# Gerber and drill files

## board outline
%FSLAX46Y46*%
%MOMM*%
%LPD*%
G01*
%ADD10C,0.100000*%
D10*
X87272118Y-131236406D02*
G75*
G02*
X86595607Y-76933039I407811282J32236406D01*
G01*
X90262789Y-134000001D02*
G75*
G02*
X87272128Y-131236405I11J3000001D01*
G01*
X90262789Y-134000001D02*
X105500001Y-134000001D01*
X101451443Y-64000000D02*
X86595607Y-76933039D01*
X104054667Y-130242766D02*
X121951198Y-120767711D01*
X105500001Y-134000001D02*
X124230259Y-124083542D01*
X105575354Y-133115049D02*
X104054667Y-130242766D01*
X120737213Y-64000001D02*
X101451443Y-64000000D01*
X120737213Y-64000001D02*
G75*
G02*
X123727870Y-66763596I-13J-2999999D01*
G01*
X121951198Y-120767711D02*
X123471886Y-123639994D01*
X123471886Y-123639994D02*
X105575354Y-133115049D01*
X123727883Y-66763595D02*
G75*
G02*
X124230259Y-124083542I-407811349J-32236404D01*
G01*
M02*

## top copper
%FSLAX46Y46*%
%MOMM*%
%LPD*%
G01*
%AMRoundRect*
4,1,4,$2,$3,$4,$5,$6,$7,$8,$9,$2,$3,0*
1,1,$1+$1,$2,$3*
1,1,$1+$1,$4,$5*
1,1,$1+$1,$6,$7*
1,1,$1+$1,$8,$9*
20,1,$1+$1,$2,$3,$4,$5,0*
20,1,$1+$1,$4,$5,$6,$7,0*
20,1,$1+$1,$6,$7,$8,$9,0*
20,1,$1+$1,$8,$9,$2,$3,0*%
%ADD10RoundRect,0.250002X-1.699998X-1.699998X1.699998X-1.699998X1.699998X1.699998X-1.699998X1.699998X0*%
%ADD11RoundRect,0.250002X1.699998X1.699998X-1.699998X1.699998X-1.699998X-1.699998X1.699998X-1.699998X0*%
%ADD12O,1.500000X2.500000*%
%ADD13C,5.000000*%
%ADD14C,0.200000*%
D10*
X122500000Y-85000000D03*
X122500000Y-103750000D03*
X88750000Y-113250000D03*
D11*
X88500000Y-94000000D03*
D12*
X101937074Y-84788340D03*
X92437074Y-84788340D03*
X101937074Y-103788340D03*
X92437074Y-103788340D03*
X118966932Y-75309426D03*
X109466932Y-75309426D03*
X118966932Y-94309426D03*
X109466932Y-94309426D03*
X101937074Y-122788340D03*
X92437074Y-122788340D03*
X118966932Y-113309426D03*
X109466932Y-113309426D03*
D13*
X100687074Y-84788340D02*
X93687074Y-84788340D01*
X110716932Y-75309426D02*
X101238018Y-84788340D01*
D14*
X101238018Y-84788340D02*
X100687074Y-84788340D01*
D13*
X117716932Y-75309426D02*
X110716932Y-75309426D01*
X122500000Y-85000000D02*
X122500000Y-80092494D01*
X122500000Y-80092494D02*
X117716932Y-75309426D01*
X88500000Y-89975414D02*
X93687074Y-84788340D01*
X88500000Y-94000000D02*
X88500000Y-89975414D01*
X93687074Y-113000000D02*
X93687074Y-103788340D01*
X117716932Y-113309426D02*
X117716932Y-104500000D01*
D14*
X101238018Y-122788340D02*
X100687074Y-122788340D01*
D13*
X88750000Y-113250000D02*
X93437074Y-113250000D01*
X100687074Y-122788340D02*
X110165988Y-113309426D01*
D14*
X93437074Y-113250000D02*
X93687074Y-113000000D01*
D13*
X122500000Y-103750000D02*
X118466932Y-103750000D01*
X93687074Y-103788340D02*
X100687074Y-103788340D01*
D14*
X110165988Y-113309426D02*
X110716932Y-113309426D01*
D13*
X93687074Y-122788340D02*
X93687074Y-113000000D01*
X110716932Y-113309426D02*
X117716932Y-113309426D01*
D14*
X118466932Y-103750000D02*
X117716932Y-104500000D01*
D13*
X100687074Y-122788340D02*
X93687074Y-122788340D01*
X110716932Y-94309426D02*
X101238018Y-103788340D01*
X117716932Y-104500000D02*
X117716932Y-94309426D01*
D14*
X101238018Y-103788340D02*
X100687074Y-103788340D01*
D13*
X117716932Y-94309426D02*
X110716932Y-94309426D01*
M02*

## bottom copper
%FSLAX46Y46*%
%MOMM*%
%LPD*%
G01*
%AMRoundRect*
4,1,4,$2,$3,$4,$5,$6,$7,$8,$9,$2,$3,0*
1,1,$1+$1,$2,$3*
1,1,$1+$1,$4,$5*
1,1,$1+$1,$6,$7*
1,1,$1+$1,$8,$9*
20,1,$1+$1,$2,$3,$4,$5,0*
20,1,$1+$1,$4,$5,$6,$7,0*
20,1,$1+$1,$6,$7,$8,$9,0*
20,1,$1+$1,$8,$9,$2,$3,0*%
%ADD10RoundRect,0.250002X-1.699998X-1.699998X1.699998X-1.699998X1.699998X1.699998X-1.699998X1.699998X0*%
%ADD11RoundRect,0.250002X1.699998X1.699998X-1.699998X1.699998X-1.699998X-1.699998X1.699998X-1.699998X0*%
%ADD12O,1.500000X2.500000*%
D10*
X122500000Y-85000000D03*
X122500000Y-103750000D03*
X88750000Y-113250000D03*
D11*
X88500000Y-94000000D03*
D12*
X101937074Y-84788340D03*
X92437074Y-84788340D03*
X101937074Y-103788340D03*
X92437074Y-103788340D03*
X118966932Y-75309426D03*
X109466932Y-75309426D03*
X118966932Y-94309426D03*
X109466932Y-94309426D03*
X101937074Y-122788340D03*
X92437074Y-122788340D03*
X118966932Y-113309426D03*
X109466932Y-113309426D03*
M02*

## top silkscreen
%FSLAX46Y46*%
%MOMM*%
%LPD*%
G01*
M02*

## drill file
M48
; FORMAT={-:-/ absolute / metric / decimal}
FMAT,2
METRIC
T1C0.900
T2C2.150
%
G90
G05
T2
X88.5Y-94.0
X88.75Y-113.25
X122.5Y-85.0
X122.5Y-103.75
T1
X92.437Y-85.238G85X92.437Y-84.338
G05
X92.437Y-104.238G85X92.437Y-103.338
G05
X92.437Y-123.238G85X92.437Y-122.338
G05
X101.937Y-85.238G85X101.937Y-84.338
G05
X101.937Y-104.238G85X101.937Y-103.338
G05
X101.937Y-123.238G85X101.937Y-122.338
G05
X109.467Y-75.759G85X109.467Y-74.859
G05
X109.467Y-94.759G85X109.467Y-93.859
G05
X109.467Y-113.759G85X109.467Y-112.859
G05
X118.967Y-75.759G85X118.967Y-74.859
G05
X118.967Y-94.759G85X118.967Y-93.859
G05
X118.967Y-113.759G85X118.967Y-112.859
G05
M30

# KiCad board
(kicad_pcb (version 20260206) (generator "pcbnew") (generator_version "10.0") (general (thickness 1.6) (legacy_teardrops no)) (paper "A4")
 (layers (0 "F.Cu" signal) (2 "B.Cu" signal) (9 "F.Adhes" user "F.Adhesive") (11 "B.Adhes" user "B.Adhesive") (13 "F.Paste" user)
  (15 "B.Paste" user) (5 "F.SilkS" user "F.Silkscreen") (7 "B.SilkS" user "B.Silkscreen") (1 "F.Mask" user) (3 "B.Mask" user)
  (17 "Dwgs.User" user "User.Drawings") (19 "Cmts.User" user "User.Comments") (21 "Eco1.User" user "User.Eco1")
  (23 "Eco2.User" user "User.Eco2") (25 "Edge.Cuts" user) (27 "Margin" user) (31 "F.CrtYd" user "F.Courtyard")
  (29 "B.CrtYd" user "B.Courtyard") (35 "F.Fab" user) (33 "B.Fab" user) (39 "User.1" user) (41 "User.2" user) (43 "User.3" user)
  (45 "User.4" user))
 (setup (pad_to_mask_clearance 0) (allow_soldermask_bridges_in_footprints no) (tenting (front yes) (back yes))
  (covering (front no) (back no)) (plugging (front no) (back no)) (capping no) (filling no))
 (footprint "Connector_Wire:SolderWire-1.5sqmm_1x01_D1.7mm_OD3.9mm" (layer "F.Cu") (at 122.5 85)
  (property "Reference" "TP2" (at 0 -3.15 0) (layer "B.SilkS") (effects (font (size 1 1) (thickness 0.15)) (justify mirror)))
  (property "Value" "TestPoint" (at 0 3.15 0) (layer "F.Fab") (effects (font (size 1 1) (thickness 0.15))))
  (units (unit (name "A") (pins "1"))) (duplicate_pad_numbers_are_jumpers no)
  (pad "1" thru_hole roundrect (at 0 0) (size 3.9 3.9) (drill 2.15) (layers "*.Cu" "*.Mask") (remove_unused_layers no)
   (roundrect_rratio 0.064103) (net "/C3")))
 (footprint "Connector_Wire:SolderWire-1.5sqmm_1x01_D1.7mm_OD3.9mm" (layer "F.Cu") (at 122.5 103.75)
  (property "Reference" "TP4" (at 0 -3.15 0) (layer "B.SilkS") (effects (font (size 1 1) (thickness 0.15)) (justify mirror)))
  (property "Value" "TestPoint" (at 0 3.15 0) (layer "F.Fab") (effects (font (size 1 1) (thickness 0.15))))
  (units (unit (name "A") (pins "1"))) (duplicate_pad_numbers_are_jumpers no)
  (pad "1" thru_hole roundrect (at 0 0) (size 3.9 3.9) (drill 2.15) (layers "*.Cu" "*.Mask") (remove_unused_layers no)
   (roundrect_rratio 0.064103) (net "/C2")))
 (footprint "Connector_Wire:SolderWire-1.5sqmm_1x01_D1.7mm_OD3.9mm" (layer "F.Cu") (at 88.75 113.25)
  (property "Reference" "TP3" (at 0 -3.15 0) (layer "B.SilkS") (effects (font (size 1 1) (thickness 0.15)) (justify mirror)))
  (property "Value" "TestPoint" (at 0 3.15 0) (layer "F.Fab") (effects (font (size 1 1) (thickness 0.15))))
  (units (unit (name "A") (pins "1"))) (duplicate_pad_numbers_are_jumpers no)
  (pad "1" thru_hole roundrect (at 0 0) (size 3.9 3.9) (drill 2.15) (layers "*.Cu" "*.Mask") (remove_unused_layers no)
   (roundrect_rratio 0.064103) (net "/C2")))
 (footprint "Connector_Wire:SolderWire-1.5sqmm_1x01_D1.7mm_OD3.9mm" (layer "B.Cu") (at 88.5 94 180)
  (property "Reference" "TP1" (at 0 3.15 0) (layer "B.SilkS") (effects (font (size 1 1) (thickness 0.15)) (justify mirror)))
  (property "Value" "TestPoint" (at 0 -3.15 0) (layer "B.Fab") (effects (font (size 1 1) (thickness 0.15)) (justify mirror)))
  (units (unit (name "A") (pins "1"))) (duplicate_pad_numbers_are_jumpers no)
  (pad "1" thru_hole roundrect (at 0 0 180) (size 3.9 3.9) (drill 2.15) (layers "*.Cu" "*.Mask") (remove_unused_layers no)
   (roundrect_rratio 0.064103) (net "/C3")))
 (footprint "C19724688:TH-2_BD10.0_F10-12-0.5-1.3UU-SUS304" (layer "B.Cu") (at 97.187074 84.78834 180)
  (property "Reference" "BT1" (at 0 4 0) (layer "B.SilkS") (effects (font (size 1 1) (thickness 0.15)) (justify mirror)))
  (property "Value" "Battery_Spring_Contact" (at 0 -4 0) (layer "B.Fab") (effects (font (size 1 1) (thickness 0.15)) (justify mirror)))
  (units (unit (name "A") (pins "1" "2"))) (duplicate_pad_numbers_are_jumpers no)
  (pad "1" thru_hole oval (at -4.75 0 180) (size 1.5 2.5) (drill oval 0.900024 1.799996) (layers "*.Cu" "*.Mask") (remove_unused_layers no)
   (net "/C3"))
  (pad "2" thru_hole oval (at 4.75 0 180) (size 1.5 2.5) (drill oval 0.900024 1.799996) (layers "*.Cu" "*.Mask") (remove_unused_layers no)
   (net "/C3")))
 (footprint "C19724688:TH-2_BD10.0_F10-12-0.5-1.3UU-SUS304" (layer "B.Cu") (at 97.187074 103.78834 180)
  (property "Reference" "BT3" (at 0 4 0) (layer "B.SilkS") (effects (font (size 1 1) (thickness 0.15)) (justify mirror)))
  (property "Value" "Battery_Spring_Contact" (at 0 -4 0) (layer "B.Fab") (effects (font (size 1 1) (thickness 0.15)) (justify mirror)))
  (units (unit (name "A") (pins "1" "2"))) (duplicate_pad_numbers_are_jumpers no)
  (pad "1" thru_hole oval (at -4.75 0 180) (size 1.5 2.5) (drill oval 0.900024 1.799996) (layers "*.Cu" "*.Mask") (remove_unused_layers no)
   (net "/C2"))
  (pad "2" thru_hole oval (at 4.75 0 180) (size 1.5 2.5) (drill oval 0.900024 1.799996) (layers "*.Cu" "*.Mask") (remove_unused_layers no)
   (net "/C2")))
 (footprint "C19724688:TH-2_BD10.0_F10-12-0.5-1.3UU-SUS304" (layer "B.Cu") (at 114.216932 75.309426 180)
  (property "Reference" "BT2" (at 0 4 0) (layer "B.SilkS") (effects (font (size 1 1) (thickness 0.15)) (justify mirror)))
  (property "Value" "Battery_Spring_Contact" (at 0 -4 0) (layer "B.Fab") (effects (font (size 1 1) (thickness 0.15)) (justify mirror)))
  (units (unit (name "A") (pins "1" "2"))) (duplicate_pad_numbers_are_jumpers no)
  (pad "1" thru_hole oval (at -4.75 0 180) (size 1.5 2.5) (drill oval 0.900024 1.799996) (layers "*.Cu" "*.Mask") (remove_unused_layers no)
   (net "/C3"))
  (pad "2" thru_hole oval (at 4.75 0 180) (size 1.5 2.5) (drill oval 0.900024 1.799996) (layers "*.Cu" "*.Mask") (remove_unused_layers no)
   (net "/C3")))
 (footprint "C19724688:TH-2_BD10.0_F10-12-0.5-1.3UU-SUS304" (layer "B.Cu") (at 114.216932 94.309426 180)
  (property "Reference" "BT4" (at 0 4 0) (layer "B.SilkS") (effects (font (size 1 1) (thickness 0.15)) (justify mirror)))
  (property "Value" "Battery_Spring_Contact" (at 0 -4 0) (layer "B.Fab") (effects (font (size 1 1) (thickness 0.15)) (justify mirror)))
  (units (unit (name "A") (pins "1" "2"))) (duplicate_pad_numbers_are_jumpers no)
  (pad "1" thru_hole oval (at -4.75 0 180) (size 1.5 2.5) (drill oval 0.900024 1.799996) (layers "*.Cu" "*.Mask") (remove_unused_layers no)
   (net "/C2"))
  (pad "2" thru_hole oval (at 4.75 0 180) (size 1.5 2.5) (drill oval 0.900024 1.799996) (layers "*.Cu" "*.Mask") (remove_unused_layers no)
   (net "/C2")))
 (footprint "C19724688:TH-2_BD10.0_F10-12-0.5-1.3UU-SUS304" (layer "B.Cu") (at 97.187074 122.78834 180)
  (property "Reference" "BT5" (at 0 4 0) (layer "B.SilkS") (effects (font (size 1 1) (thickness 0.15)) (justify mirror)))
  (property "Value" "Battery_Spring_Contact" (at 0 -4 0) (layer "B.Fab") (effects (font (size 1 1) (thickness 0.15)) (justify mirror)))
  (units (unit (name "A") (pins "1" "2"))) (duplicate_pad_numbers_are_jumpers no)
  (pad "1" thru_hole oval (at -4.75 0 180) (size 1.5 2.5) (drill oval 0.900024 1.799996) (layers "*.Cu" "*.Mask") (remove_unused_layers no)
   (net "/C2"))
  (pad "2" thru_hole oval (at 4.75 0 180) (size 1.5 2.5) (drill oval 0.900024 1.799996) (layers "*.Cu" "*.Mask") (remove_unused_layers no)
   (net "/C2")))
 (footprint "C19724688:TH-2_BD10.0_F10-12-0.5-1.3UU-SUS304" (layer "B.Cu") (at 114.216932 113.309426 180)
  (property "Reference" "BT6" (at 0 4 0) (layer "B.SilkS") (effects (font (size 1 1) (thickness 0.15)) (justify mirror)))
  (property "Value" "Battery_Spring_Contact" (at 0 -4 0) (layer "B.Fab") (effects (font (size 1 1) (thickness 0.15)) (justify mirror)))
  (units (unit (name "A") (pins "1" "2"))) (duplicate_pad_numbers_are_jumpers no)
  (pad "1" thru_hole oval (at -4.75 0 180) (size 1.5 2.5) (drill oval 0.900024 1.799996) (layers "*.Cu" "*.Mask") (remove_unused_layers no)
   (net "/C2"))
  (pad "2" thru_hole oval (at 4.75 0 180) (size 1.5 2.5) (drill oval 0.900024 1.799996) (layers "*.Cu" "*.Mask") (remove_unused_layers no)
   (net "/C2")))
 (gr_arc (start 87.272118 131.236406) (mid 86.031742 104.095961) (end 86.595607 76.933039) (stroke (width 0.1) (type default))
  (layer "Edge.Cuts"))
 (gr_arc (start 90.262789 134.000001) (mid 88.226767 133.203318) (end 87.272118 131.236406) (stroke (width 0.1) (type default))
  (layer "Edge.Cuts"))
 (gr_line (start 90.262789 134.000001) (end 105.500001 134.000001) (stroke (width 0.1) (type default)) (layer "Edge.Cuts"))
 (gr_line (start 101.451443 64) (end 86.595607 76.933039) (stroke (width 0.1) (type default)) (layer "Edge.Cuts"))
 (gr_line (start 104.054667 130.242766) (end 121.951198 120.767711) (stroke (width 0.1) (type default)) (layer "Edge.Cuts"))
 (gr_line (start 105.500001 134.000001) (end 124.230259 124.083542) (stroke (width 0.1) (type default)) (layer "Edge.Cuts"))
 (gr_line (start 105.575354 133.115049) (end 104.054667 130.242766) (stroke (width 0.1) (type default)) (layer "Edge.Cuts"))
 (gr_line (start 120.737213 64.000001) (end 101.451443 64) (stroke (width 0.1) (type default)) (layer "Edge.Cuts"))
 (gr_arc (start 120.737213 64.000001) (mid 122.773235 64.796684) (end 123.727883 66.763595) (stroke (width 0.1) (type default))
  (layer "Edge.Cuts"))
 (gr_line (start 121.951198 120.767711) (end 123.471886 123.639994) (stroke (width 0.1) (type default)) (layer "Edge.Cuts"))
 (gr_line (start 123.471886 123.639994) (end 105.575354 133.115049) (stroke (width 0.1) (type default)) (layer "Edge.Cuts"))
 (gr_arc (start 123.727883 66.763595) (mid 124.984289 95.414758) (end 124.230259 124.083542) (stroke (width 0.1) (type default))
  (layer "Edge.Cuts"))
 (segment (start 100.687074 84.78834) (end 93.687074 84.78834) (width 5) (layer "F.Cu") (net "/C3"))
 (segment (start 110.716932 75.309426) (end 101.238018 84.78834) (width 5) (layer "F.Cu") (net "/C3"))
 (segment (start 101.238018 84.78834) (end 100.687074 84.78834) (width 0.2) (layer "F.Cu") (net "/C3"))
 (segment (start 117.716932 75.309426) (end 110.716932 75.309426) (width 5) (layer "F.Cu") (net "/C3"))
 (segment (start 122.5 85) (end 122.5 80.092494) (width 5) (layer "F.Cu") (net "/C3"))
 (segment (start 122.5 80.092494) (end 117.716932 75.309426) (width 5) (layer "F.Cu") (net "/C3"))
 (segment (start 88.5 89.975414) (end 93.687074 84.78834) (width 5) (layer "F.Cu") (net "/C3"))
 (segment (start 88.5 94) (end 88.5 89.975414) (width 5) (layer "F.Cu") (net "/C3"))
 (segment (start 93.687074 113) (end 93.687074 103.78834) (width 5) (layer "F.Cu") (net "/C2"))
 (segment (start 117.716932 113.309426) (end 117.716932 104.5) (width 5) (layer "F.Cu") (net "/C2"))
 (segment (start 101.238018 122.78834) (end 100.687074 122.78834) (width 0.2) (layer "F.Cu") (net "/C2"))
 (segment (start 88.75 113.25) (end 93.437074 113.25) (width 5) (layer "F.Cu") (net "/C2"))
 (segment (start 100.687074 122.78834) (end 110.165988 113.309426) (width 5) (layer "F.Cu") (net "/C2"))
 (segment (start 93.437074 113.25) (end 93.687074 113) (width 0.2) (layer "F.Cu") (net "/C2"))
 (segment (start 122.5 103.75) (end 118.466932 103.75) (width 5) (layer "F.Cu") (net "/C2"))
 (segment (start 93.687074 103.78834) (end 100.687074 103.78834) (width 5) (layer "F.Cu") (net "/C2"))
 (segment (start 110.165988 113.309426) (end 110.716932 113.309426) (width 0.2) (layer "F.Cu") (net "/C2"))
 (segment (start 93.687074 122.78834) (end 93.687074 113) (width 5) (layer "F.Cu") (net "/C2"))
 (segment (start 110.716932 113.309426) (end 117.716932 113.309426) (width 5) (layer "F.Cu") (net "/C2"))
 (segment (start 118.466932 103.75) (end 117.716932 104.5) (width 0.2) (layer "F.Cu") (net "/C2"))
 (segment (start 100.687074 122.78834) (end 93.687074 122.78834) (width 5) (layer "F.Cu") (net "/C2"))
 (segment (start 110.716932 94.309426) (end 101.238018 103.78834) (width 5) (layer "F.Cu") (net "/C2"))
 (segment (start 117.716932 104.5) (end 117.716932 94.309426) (width 5) (layer "F.Cu") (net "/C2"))
 (segment (start 101.238018 103.78834) (end 100.687074 103.78834) (width 0.2) (layer "F.Cu") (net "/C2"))
 (segment (start 117.716932 94.309426) (end 110.716932 94.309426) (width 5) (layer "F.Cu") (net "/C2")))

